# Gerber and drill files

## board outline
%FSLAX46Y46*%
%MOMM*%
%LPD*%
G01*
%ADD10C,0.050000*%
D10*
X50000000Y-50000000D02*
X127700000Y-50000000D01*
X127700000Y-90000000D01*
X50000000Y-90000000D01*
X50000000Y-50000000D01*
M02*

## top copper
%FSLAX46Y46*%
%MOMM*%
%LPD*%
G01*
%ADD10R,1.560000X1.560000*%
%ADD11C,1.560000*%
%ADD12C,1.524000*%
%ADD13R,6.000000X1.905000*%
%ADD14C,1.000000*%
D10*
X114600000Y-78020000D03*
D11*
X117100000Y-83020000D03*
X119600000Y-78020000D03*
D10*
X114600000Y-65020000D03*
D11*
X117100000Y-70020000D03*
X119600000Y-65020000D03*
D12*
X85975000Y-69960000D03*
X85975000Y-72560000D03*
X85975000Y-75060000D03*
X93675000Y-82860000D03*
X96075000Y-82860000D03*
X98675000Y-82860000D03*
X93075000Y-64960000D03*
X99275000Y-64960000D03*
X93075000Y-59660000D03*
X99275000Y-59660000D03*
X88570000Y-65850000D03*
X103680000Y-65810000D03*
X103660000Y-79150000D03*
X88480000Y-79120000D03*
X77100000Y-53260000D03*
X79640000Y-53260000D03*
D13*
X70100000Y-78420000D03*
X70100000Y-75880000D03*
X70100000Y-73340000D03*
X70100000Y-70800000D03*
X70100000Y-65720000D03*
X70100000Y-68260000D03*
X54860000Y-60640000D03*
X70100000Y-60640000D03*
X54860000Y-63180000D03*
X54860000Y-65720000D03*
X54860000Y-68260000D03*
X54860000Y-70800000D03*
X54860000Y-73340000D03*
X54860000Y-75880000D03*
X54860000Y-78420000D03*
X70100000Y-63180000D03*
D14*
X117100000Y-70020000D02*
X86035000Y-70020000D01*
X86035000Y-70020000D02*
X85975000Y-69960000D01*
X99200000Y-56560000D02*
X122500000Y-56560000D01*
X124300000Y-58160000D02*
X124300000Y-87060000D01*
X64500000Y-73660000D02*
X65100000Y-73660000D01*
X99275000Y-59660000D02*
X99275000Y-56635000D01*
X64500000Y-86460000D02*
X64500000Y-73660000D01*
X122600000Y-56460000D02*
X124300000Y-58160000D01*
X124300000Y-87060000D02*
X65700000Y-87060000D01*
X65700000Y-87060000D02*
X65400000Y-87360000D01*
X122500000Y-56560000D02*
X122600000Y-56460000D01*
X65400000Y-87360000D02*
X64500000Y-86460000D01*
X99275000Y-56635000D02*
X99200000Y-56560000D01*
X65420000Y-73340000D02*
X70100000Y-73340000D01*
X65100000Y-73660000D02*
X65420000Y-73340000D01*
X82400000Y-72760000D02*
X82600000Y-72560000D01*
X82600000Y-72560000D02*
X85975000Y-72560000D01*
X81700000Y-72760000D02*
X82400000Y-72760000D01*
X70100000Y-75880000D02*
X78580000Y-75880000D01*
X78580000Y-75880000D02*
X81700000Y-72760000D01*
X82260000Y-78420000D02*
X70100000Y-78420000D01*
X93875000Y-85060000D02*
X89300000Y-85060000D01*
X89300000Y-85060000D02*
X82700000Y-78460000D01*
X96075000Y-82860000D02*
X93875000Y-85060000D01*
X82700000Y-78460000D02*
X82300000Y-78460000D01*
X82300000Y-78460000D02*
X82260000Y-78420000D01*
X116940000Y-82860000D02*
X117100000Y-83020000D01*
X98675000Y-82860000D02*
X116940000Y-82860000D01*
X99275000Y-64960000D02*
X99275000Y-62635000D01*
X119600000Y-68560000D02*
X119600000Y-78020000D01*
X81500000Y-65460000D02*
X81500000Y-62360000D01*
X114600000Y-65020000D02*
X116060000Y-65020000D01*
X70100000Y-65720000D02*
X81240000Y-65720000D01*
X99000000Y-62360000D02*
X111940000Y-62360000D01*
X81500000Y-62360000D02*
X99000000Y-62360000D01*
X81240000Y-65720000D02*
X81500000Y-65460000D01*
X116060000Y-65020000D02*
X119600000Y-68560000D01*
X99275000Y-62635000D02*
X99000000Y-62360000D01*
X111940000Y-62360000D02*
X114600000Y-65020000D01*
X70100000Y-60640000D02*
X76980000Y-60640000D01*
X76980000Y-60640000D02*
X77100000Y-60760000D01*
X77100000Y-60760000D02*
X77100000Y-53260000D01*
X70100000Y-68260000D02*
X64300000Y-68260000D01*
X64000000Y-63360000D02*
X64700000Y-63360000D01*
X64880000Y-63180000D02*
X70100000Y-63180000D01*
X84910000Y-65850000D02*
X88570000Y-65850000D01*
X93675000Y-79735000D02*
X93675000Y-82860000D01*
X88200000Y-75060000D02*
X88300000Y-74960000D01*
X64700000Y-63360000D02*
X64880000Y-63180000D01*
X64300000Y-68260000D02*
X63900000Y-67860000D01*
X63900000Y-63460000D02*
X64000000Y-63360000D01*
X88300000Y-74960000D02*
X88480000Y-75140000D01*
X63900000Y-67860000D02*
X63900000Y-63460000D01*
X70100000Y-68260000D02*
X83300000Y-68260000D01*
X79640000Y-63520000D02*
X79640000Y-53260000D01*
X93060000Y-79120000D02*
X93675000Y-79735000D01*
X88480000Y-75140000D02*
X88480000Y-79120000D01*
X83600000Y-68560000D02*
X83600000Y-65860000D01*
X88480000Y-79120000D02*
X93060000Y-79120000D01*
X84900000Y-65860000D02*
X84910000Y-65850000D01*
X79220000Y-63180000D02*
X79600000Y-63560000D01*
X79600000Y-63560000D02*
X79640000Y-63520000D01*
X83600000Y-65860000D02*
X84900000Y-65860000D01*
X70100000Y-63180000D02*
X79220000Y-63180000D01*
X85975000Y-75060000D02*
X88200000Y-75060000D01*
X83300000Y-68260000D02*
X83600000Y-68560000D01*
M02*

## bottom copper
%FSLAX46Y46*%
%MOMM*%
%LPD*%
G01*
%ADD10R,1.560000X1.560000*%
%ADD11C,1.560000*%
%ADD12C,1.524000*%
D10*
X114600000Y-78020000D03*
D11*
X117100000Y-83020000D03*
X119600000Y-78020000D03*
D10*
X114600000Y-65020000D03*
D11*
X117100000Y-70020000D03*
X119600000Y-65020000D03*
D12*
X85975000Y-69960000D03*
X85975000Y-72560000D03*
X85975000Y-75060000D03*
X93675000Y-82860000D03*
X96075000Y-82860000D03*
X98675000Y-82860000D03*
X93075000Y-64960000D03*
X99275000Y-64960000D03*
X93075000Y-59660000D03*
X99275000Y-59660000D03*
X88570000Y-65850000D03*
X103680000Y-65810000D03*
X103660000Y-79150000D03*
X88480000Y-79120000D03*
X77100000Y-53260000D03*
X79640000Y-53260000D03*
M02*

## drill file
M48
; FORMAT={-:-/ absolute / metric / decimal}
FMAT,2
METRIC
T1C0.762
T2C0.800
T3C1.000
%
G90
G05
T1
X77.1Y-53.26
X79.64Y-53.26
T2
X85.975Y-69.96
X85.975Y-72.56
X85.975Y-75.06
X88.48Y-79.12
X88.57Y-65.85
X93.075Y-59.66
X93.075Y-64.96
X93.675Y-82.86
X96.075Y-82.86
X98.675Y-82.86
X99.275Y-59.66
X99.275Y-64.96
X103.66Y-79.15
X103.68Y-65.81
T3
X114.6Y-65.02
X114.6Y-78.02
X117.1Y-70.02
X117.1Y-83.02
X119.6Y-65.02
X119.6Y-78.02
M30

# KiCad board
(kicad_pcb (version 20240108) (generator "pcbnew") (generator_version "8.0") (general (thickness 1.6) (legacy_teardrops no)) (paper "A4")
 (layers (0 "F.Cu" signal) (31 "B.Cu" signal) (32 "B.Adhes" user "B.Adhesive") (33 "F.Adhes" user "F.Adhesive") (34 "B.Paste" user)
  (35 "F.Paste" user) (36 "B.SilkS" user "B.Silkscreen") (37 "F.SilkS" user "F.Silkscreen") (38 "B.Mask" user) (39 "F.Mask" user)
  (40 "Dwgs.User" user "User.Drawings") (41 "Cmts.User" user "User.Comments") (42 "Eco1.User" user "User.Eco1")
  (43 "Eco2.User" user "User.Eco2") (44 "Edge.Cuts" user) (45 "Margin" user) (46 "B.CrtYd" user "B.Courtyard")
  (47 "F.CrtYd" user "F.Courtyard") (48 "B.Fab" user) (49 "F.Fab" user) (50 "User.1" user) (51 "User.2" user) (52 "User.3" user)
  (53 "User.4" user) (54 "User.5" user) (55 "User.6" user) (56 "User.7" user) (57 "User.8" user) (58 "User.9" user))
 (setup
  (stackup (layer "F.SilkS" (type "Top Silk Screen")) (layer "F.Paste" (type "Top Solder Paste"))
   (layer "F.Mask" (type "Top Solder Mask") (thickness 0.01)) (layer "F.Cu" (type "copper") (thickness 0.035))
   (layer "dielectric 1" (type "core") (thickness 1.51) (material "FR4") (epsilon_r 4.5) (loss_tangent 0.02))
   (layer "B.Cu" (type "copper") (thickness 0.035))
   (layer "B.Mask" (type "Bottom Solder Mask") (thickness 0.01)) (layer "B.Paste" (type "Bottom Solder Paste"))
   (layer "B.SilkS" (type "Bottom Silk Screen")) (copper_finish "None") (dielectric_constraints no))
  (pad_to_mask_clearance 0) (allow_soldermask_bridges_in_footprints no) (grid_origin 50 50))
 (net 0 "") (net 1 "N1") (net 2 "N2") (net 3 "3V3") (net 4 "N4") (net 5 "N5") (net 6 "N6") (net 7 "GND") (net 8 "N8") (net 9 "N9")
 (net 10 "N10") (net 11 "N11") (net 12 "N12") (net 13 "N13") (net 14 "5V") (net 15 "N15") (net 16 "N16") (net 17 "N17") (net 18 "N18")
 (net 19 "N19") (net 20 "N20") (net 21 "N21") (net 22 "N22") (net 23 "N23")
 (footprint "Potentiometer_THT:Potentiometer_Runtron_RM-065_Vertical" (layer "F.Cu") (at 114.6 78.02)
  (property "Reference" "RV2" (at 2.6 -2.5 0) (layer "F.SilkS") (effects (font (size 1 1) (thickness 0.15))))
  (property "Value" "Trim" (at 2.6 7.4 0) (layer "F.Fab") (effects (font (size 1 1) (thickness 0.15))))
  (pad "1" thru_hole rect (at 0 0) (size 1.56 1.56) (drill 1) (layers "*.Cu" "*.Mask") (remove_unused_layers no) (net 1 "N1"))
  (pad "2" thru_hole circle (at 2.5 5) (size 1.56 1.56) (drill 1) (layers "*.Cu" "*.Mask") (remove_unused_layers no) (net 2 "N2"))
  (pad "3" thru_hole circle (at 5 0) (size 1.56 1.56) (drill 1) (layers "*.Cu" "*.Mask") (remove_unused_layers no) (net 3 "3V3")))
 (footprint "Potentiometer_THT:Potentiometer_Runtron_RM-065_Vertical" (layer "F.Cu") (at 114.6 65.02)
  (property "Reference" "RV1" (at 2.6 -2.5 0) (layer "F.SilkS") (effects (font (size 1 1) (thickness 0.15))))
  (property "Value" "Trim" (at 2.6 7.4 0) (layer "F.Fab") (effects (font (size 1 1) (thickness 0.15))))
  (pad "1" thru_hole rect (at 0 0) (size 1.56 1.56) (drill 1) (layers "*.Cu" "*.Mask") (remove_unused_layers no) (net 3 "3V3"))
  (pad "2" thru_hole circle (at 2.5 5) (size 1.56 1.56) (drill 1) (layers "*.Cu" "*.Mask") (remove_unused_layers no) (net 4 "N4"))
  (pad "3" thru_hole circle (at 5 0) (size 1.56 1.56) (drill 1) (layers "*.Cu" "*.Mask") (remove_unused_layers no) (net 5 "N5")))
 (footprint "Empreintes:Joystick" (layer "F.Cu") (at 96.1 71.26)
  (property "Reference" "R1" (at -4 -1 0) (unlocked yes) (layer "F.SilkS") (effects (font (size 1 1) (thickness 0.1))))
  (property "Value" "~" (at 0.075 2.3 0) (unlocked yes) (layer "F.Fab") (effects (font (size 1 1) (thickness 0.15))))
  (pad "1" thru_hole circle (at -10.125 -1.3) (size 1.524 1.524) (drill 0.8) (layers "*.Cu" "*.Mask") (remove_unused_layers no) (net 4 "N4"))
  (pad "2" thru_hole circle (at -10.125 1.3) (size 1.524 1.524) (drill 0.8) (layers "*.Cu" "*.Mask") (remove_unused_layers no) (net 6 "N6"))
  (pad "3" thru_hole circle (at -10.125 3.8) (size 1.524 1.524) (drill 0.8) (layers "*.Cu" "*.Mask") (remove_unused_layers no) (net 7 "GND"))
  (pad "4" thru_hole circle (at -2.425 11.6) (size 1.524 1.524) (drill 0.8) (layers "*.Cu" "*.Mask") (remove_unused_layers no) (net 7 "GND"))
  (pad "5" thru_hole circle (at -0.025 11.6) (size 1.524 1.524) (drill 0.8) (layers "*.Cu" "*.Mask") (remove_unused_layers no) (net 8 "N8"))
  (pad "6" thru_hole circle (at 2.575 11.6) (size 1.524 1.524) (drill 0.8) (layers "*.Cu" "*.Mask") (remove_unused_layers no) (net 2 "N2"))
  (pad "7" thru_hole circle (at -3.025 -6.3) (size 1.524 1.524) (drill 0.8) (layers "*.Cu" "*.Mask") (remove_unused_layers no) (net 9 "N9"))
  (pad "8" thru_hole circle (at 3.175 -6.3) (size 1.524 1.524) (drill 0.8) (layers "*.Cu" "*.Mask") (remove_unused_layers no) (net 3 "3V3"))
  (pad "9" thru_hole circle (at -3.025 -11.6) (size 1.524 1.524) (drill 0.8) (layers "*.Cu" "*.Mask") (remove_unused_layers no)
   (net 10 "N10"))
  (pad "10" thru_hole circle (at 3.175 -11.6) (size 1.524 1.524) (drill 0.8) (layers "*.Cu" "*.Mask") (remove_unused_layers no)
   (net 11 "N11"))
  (pad "11" thru_hole circle (at -7.53 -5.41) (size 1.524 1.524) (drill 0.8) (layers "*.Cu" "*.Mask") (remove_unused_layers no)
   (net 7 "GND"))
  (pad "12" thru_hole circle (at 7.58 -5.45) (size 1.524 1.524) (drill 0.8) (layers "*.Cu" "*.Mask") (remove_unused_layers no)
   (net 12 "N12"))
  (pad "13" thru_hole circle (at 7.56 7.89) (size 1.524 1.524) (drill 0.8) (layers "*.Cu" "*.Mask") (remove_unused_layers no) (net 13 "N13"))
  (pad "14" thru_hole circle (at -7.62 7.86) (size 1.524 1.524) (drill 0.8) (layers "*.Cu" "*.Mask") (remove_unused_layers no) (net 7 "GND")))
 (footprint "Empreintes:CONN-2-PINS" (layer "F.Cu") (at 78.37 53.26)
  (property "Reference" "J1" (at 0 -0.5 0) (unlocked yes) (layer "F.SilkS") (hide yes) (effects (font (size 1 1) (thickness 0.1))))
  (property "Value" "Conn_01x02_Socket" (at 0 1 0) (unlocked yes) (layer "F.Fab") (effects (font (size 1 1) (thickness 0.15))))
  (pad "1" thru_hole circle (at -1.27 0) (size 1.524 1.524) (drill 0.762) (layers "*.Cu" "*.Mask") (remove_unused_layers no) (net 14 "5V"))
  (pad "2" thru_hole circle (at 1.27 0) (size 1.524 1.524) (drill 0.762) (layers "*.Cu" "*.Mask") (remove_unused_layers no) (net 7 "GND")))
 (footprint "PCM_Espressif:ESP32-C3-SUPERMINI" (layer "F.Cu") (at 62.48 70.54)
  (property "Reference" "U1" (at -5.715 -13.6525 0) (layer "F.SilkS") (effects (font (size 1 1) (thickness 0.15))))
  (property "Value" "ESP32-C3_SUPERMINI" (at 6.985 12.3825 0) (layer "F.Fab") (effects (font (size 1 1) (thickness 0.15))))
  (pad "0" smd rect (at 7.62 7.88) (size 6 1.905) (layers "F.Cu" "F.Paste" "F.Mask") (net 8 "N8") (solder_mask_margin 0.102))
  (pad "1" smd rect (at 7.62 5.34) (size 6 1.905) (layers "F.Cu" "F.Paste" "F.Mask") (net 6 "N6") (solder_mask_margin 0.102))
  (pad "2" smd rect (at 7.62 2.8) (size 6 1.905) (layers "F.Cu" "F.Paste" "F.Mask") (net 11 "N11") (solder_mask_margin 0.102))
  (pad "3" smd rect (at 7.62 0.26) (size 6 1.905) (layers "F.Cu" "F.Paste" "F.Mask") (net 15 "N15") (solder_mask_margin 0.102))
  (pad "3.3" smd rect (at 7.62 -4.82) (size 6 1.905) (layers "F.Cu" "F.Paste" "F.Mask") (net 3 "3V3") (solder_mask_margin 0.102))
  (pad "4" smd rect (at 7.62 -2.28) (size 6 1.905) (layers "F.Cu" "F.Paste" "F.Mask") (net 7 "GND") (solder_mask_margin 0.102))
  (pad "5" smd rect (at -7.62 -9.9) (size 6 1.905) (layers "F.Cu" "F.Paste" "F.Mask") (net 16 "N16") (solder_mask_margin 0.102))
  (pad "5V" smd rect (at 7.62 -9.9) (size 6 1.905) (layers "F.Cu" "F.Paste" "F.Mask") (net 14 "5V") (solder_mask_margin 0.102))
  (pad "6" smd rect (at -7.62 -7.36) (size 6 1.905) (layers "F.Cu" "F.Paste" "F.Mask") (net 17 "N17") (solder_mask_margin 0.102))
  (pad "7" smd rect (at -7.62 -4.82) (size 6 1.905) (layers "F.Cu" "F.Paste" "F.Mask") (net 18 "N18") (solder_mask_margin 0.102))
  (pad "8" smd rect (at -7.62 -2.28) (size 6 1.905) (layers "F.Cu" "F.Paste" "F.Mask") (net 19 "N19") (solder_mask_margin 0.102))
  (pad "9" smd rect (at -7.62 0.26) (size 6 1.905) (layers "F.Cu" "F.Paste" "F.Mask") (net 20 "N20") (solder_mask_margin 0.102))
  (pad "10" smd rect (at -7.62 2.8) (size 6 1.905) (layers "F.Cu" "F.Paste" "F.Mask") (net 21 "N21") (solder_mask_margin 0.102))
  (pad "20" smd rect (at -7.62 5.34) (size 6 1.905) (layers "F.Cu" "F.Paste" "F.Mask") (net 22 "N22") (solder_mask_margin 0.102))
  (pad "21" smd rect (at -7.62 7.88) (size 6 1.905) (layers "F.Cu" "F.Paste" "F.Mask") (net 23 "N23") (solder_mask_margin 0.102))
  (pad "G" smd rect (at 7.62 -7.36) (size 6 1.905) (layers "F.Cu" "F.Paste" "F.Mask") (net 7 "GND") (solder_mask_margin 0.102)))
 (gr_rect (start 50 50) (end 127.7 90) (stroke (width 0.05) (type default)) (fill none) (layer "Edge.Cuts"))
 (segment (start 117.1 70.02) (end 86.035 70.02) (width 1) (layer "F.Cu") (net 4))
 (segment (start 86.035 70.02) (end 85.975 69.96) (width 1) (layer "F.Cu") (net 4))
 (segment (start 99.2 56.56) (end 122.5 56.56) (width 1) (layer "F.Cu") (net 11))
 (segment (start 124.3 58.16) (end 124.3 87.06) (width 1) (layer "F.Cu") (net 11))
 (segment (start 64.5 73.66) (end 65.1 73.66) (width 1) (layer "F.Cu") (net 11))
 (segment (start 99.275 59.66) (end 99.275 56.635) (width 1) (layer "F.Cu") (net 11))
 (segment (start 64.5 86.46) (end 64.5 73.66) (width 1) (layer "F.Cu") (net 11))
 (segment (start 122.6 56.46) (end 124.3 58.16) (width 1) (layer "F.Cu") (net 11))
 (segment (start 124.3 87.06) (end 65.7 87.06) (width 1) (layer "F.Cu") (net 11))
 (segment (start 65.7 87.06) (end 65.4 87.36) (width 1) (layer "F.Cu") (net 11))
 (segment (start 122.5 56.56) (end 122.6 56.46) (width 1) (layer "F.Cu") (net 11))
 (segment (start 65.4 87.36) (end 64.5 86.46) (width 1) (layer "F.Cu") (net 11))
 (segment (start 99.275 56.635) (end 99.2 56.56) (width 1) (layer "F.Cu") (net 11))
 (segment (start 65.42 73.34) (end 70.1 73.34) (width 1) (layer "F.Cu") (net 11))
 (segment (start 65.1 73.66) (end 65.42 73.34) (width 1) (layer "F.Cu") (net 11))
 (segment (start 82.4 72.76) (end 82.6 72.56) (width 1) (layer "F.Cu") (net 6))
 (segment (start 82.6 72.56) (end 85.975 72.56) (width 1) (layer "F.Cu") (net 6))
 (segment (start 81.7 72.76) (end 82.4 72.76) (width 1) (layer "F.Cu") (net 6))
 (segment (start 70.1 75.88) (end 78.58 75.88) (width 1) (layer "F.Cu") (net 6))
 (segment (start 78.58 75.88) (end 81.7 72.76) (width 1) (layer "F.Cu") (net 6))
 (segment (start 82.26 78.42) (end 70.1 78.42) (width 1) (layer "F.Cu") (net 8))
 (segment (start 93.875 85.06) (end 89.3 85.06) (width 1) (layer "F.Cu") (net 8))
 (segment (start 89.3 85.06) (end 82.7 78.46) (width 1) (layer "F.Cu") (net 8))
 (segment (start 96.075 82.86) (end 93.875 85.06) (width 1) (layer "F.Cu") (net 8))
 (segment (start 82.7 78.46) (end 82.3 78.46) (width 1) (layer "F.Cu") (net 8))
 (segment (start 82.3 78.46) (end 82.26 78.42) (width 1) (layer "F.Cu") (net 8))
 (segment (start 116.94 82.86) (end 117.1 83.02) (width 1) (layer "F.Cu") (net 2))
 (segment (start 98.675 82.86) (end 116.94 82.86) (width 1) (layer "F.Cu") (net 2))
 (segment (start 99.275 64.96) (end 99.275 62.635) (width 1) (layer "F.Cu") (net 3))
 (segment (start 119.6 68.56) (end 119.6 78.02) (width 1) (layer "F.Cu") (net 3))
 (segment (start 81.5 65.46) (end 81.5 62.36) (width 1) (layer "F.Cu") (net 3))
 (segment (start 114.6 65.02) (end 116.06 65.02) (width 1) (layer "F.Cu") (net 3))
 (segment (start 70.1 65.72) (end 81.24 65.72) (width 1) (layer "F.Cu") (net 3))
 (segment (start 99 62.36) (end 111.94 62.36) (width 1) (layer "F.Cu") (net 3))
 (segment (start 81.5 62.36) (end 99 62.36) (width 1) (layer "F.Cu") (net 3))
 (segment (start 81.24 65.72) (end 81.5 65.46) (width 1) (layer "F.Cu") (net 3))
 (segment (start 116.06 65.02) (end 119.6 68.56) (width 1) (layer "F.Cu") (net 3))
 (segment (start 99.275 62.635) (end 99 62.36) (width 1) (layer "F.Cu") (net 3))
 (segment (start 111.94 62.36) (end 114.6 65.02) (width 1) (layer "F.Cu") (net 3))
 (segment (start 70.1 60.64) (end 76.98 60.64) (width 1) (layer "F.Cu") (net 14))
 (segment (start 76.98 60.64) (end 77.1 60.76) (width 1) (layer "F.Cu") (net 14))
 (segment (start 77.1 60.76) (end 77.1 53.26) (width 1) (layer "F.Cu") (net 14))
 (segment (start 70.1 68.26) (end 64.3 68.26) (width 1) (layer "F.Cu") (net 7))
 (segment (start 64 63.36) (end 64.7 63.36) (width 1) (layer "F.Cu") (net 7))
 (segment (start 64.88 63.18) (end 70.1 63.18) (width 1) (layer "F.Cu") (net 7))
 (segment (start 84.91 65.85) (end 88.57 65.85) (width 1) (layer "F.Cu") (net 7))
 (segment (start 93.675 79.735) (end 93.675 82.86) (width 1) (layer "F.Cu") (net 7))
 (segment (start 88.2 75.06) (end 88.3 74.96) (width 1) (layer "F.Cu") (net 7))
 (segment (start 64.7 63.36) (end 64.88 63.18) (width 1) (layer "F.Cu") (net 7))
 (segment (start 64.3 68.26) (end 63.9 67.86) (width 1) (layer "F.Cu") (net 7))
 (segment (start 63.9 63.46) (end 64 63.36) (width 1) (layer "F.Cu") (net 7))
 (segment (start 88.3 74.96) (end 88.48 75.14) (width 1) (layer "F.Cu") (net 7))
 (segment (start 63.9 67.86) (end 63.9 63.46) (width 1) (layer "F.Cu") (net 7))
 (segment (start 70.1 68.26) (end 83.3 68.26) (width 1) (layer "F.Cu") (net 7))
 (segment (start 79.64 63.52) (end 79.64 53.26) (width 1) (layer "F.Cu") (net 7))
 (segment (start 93.06 79.12) (end 93.675 79.735) (width 1) (layer "F.Cu") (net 7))
 (segment (start 88.48 75.14) (end 88.48 79.12) (width 1) (layer "F.Cu") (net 7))
 (segment (start 83.6 68.56) (end 83.6 65.86) (width 1) (layer "F.Cu") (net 7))
 (segment (start 88.48 79.12) (end 93.06 79.12) (width 1) (layer "F.Cu") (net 7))
 (segment (start 84.9 65.86) (end 84.91 65.85) (width 1) (layer "F.Cu") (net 7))
 (segment (start 79.22 63.18) (end 79.6 63.56) (width 1) (layer "F.Cu") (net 7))
 (segment (start 79.6 63.56) (end 79.64 63.52) (width 1) (layer "F.Cu") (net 7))
 (segment (start 83.6 65.86) (end 84.9 65.86) (width 1) (layer "F.Cu") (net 7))
 (segment (start 70.1 63.18) (end 79.22 63.18) (width 1) (layer "F.Cu") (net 7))
 (segment (start 85.975 75.06) (end 88.2 75.06) (width 1) (layer "F.Cu") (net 7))
 (segment (start 83.3 68.26) (end 83.6 68.56) (width 1) (layer "F.Cu") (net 7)))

